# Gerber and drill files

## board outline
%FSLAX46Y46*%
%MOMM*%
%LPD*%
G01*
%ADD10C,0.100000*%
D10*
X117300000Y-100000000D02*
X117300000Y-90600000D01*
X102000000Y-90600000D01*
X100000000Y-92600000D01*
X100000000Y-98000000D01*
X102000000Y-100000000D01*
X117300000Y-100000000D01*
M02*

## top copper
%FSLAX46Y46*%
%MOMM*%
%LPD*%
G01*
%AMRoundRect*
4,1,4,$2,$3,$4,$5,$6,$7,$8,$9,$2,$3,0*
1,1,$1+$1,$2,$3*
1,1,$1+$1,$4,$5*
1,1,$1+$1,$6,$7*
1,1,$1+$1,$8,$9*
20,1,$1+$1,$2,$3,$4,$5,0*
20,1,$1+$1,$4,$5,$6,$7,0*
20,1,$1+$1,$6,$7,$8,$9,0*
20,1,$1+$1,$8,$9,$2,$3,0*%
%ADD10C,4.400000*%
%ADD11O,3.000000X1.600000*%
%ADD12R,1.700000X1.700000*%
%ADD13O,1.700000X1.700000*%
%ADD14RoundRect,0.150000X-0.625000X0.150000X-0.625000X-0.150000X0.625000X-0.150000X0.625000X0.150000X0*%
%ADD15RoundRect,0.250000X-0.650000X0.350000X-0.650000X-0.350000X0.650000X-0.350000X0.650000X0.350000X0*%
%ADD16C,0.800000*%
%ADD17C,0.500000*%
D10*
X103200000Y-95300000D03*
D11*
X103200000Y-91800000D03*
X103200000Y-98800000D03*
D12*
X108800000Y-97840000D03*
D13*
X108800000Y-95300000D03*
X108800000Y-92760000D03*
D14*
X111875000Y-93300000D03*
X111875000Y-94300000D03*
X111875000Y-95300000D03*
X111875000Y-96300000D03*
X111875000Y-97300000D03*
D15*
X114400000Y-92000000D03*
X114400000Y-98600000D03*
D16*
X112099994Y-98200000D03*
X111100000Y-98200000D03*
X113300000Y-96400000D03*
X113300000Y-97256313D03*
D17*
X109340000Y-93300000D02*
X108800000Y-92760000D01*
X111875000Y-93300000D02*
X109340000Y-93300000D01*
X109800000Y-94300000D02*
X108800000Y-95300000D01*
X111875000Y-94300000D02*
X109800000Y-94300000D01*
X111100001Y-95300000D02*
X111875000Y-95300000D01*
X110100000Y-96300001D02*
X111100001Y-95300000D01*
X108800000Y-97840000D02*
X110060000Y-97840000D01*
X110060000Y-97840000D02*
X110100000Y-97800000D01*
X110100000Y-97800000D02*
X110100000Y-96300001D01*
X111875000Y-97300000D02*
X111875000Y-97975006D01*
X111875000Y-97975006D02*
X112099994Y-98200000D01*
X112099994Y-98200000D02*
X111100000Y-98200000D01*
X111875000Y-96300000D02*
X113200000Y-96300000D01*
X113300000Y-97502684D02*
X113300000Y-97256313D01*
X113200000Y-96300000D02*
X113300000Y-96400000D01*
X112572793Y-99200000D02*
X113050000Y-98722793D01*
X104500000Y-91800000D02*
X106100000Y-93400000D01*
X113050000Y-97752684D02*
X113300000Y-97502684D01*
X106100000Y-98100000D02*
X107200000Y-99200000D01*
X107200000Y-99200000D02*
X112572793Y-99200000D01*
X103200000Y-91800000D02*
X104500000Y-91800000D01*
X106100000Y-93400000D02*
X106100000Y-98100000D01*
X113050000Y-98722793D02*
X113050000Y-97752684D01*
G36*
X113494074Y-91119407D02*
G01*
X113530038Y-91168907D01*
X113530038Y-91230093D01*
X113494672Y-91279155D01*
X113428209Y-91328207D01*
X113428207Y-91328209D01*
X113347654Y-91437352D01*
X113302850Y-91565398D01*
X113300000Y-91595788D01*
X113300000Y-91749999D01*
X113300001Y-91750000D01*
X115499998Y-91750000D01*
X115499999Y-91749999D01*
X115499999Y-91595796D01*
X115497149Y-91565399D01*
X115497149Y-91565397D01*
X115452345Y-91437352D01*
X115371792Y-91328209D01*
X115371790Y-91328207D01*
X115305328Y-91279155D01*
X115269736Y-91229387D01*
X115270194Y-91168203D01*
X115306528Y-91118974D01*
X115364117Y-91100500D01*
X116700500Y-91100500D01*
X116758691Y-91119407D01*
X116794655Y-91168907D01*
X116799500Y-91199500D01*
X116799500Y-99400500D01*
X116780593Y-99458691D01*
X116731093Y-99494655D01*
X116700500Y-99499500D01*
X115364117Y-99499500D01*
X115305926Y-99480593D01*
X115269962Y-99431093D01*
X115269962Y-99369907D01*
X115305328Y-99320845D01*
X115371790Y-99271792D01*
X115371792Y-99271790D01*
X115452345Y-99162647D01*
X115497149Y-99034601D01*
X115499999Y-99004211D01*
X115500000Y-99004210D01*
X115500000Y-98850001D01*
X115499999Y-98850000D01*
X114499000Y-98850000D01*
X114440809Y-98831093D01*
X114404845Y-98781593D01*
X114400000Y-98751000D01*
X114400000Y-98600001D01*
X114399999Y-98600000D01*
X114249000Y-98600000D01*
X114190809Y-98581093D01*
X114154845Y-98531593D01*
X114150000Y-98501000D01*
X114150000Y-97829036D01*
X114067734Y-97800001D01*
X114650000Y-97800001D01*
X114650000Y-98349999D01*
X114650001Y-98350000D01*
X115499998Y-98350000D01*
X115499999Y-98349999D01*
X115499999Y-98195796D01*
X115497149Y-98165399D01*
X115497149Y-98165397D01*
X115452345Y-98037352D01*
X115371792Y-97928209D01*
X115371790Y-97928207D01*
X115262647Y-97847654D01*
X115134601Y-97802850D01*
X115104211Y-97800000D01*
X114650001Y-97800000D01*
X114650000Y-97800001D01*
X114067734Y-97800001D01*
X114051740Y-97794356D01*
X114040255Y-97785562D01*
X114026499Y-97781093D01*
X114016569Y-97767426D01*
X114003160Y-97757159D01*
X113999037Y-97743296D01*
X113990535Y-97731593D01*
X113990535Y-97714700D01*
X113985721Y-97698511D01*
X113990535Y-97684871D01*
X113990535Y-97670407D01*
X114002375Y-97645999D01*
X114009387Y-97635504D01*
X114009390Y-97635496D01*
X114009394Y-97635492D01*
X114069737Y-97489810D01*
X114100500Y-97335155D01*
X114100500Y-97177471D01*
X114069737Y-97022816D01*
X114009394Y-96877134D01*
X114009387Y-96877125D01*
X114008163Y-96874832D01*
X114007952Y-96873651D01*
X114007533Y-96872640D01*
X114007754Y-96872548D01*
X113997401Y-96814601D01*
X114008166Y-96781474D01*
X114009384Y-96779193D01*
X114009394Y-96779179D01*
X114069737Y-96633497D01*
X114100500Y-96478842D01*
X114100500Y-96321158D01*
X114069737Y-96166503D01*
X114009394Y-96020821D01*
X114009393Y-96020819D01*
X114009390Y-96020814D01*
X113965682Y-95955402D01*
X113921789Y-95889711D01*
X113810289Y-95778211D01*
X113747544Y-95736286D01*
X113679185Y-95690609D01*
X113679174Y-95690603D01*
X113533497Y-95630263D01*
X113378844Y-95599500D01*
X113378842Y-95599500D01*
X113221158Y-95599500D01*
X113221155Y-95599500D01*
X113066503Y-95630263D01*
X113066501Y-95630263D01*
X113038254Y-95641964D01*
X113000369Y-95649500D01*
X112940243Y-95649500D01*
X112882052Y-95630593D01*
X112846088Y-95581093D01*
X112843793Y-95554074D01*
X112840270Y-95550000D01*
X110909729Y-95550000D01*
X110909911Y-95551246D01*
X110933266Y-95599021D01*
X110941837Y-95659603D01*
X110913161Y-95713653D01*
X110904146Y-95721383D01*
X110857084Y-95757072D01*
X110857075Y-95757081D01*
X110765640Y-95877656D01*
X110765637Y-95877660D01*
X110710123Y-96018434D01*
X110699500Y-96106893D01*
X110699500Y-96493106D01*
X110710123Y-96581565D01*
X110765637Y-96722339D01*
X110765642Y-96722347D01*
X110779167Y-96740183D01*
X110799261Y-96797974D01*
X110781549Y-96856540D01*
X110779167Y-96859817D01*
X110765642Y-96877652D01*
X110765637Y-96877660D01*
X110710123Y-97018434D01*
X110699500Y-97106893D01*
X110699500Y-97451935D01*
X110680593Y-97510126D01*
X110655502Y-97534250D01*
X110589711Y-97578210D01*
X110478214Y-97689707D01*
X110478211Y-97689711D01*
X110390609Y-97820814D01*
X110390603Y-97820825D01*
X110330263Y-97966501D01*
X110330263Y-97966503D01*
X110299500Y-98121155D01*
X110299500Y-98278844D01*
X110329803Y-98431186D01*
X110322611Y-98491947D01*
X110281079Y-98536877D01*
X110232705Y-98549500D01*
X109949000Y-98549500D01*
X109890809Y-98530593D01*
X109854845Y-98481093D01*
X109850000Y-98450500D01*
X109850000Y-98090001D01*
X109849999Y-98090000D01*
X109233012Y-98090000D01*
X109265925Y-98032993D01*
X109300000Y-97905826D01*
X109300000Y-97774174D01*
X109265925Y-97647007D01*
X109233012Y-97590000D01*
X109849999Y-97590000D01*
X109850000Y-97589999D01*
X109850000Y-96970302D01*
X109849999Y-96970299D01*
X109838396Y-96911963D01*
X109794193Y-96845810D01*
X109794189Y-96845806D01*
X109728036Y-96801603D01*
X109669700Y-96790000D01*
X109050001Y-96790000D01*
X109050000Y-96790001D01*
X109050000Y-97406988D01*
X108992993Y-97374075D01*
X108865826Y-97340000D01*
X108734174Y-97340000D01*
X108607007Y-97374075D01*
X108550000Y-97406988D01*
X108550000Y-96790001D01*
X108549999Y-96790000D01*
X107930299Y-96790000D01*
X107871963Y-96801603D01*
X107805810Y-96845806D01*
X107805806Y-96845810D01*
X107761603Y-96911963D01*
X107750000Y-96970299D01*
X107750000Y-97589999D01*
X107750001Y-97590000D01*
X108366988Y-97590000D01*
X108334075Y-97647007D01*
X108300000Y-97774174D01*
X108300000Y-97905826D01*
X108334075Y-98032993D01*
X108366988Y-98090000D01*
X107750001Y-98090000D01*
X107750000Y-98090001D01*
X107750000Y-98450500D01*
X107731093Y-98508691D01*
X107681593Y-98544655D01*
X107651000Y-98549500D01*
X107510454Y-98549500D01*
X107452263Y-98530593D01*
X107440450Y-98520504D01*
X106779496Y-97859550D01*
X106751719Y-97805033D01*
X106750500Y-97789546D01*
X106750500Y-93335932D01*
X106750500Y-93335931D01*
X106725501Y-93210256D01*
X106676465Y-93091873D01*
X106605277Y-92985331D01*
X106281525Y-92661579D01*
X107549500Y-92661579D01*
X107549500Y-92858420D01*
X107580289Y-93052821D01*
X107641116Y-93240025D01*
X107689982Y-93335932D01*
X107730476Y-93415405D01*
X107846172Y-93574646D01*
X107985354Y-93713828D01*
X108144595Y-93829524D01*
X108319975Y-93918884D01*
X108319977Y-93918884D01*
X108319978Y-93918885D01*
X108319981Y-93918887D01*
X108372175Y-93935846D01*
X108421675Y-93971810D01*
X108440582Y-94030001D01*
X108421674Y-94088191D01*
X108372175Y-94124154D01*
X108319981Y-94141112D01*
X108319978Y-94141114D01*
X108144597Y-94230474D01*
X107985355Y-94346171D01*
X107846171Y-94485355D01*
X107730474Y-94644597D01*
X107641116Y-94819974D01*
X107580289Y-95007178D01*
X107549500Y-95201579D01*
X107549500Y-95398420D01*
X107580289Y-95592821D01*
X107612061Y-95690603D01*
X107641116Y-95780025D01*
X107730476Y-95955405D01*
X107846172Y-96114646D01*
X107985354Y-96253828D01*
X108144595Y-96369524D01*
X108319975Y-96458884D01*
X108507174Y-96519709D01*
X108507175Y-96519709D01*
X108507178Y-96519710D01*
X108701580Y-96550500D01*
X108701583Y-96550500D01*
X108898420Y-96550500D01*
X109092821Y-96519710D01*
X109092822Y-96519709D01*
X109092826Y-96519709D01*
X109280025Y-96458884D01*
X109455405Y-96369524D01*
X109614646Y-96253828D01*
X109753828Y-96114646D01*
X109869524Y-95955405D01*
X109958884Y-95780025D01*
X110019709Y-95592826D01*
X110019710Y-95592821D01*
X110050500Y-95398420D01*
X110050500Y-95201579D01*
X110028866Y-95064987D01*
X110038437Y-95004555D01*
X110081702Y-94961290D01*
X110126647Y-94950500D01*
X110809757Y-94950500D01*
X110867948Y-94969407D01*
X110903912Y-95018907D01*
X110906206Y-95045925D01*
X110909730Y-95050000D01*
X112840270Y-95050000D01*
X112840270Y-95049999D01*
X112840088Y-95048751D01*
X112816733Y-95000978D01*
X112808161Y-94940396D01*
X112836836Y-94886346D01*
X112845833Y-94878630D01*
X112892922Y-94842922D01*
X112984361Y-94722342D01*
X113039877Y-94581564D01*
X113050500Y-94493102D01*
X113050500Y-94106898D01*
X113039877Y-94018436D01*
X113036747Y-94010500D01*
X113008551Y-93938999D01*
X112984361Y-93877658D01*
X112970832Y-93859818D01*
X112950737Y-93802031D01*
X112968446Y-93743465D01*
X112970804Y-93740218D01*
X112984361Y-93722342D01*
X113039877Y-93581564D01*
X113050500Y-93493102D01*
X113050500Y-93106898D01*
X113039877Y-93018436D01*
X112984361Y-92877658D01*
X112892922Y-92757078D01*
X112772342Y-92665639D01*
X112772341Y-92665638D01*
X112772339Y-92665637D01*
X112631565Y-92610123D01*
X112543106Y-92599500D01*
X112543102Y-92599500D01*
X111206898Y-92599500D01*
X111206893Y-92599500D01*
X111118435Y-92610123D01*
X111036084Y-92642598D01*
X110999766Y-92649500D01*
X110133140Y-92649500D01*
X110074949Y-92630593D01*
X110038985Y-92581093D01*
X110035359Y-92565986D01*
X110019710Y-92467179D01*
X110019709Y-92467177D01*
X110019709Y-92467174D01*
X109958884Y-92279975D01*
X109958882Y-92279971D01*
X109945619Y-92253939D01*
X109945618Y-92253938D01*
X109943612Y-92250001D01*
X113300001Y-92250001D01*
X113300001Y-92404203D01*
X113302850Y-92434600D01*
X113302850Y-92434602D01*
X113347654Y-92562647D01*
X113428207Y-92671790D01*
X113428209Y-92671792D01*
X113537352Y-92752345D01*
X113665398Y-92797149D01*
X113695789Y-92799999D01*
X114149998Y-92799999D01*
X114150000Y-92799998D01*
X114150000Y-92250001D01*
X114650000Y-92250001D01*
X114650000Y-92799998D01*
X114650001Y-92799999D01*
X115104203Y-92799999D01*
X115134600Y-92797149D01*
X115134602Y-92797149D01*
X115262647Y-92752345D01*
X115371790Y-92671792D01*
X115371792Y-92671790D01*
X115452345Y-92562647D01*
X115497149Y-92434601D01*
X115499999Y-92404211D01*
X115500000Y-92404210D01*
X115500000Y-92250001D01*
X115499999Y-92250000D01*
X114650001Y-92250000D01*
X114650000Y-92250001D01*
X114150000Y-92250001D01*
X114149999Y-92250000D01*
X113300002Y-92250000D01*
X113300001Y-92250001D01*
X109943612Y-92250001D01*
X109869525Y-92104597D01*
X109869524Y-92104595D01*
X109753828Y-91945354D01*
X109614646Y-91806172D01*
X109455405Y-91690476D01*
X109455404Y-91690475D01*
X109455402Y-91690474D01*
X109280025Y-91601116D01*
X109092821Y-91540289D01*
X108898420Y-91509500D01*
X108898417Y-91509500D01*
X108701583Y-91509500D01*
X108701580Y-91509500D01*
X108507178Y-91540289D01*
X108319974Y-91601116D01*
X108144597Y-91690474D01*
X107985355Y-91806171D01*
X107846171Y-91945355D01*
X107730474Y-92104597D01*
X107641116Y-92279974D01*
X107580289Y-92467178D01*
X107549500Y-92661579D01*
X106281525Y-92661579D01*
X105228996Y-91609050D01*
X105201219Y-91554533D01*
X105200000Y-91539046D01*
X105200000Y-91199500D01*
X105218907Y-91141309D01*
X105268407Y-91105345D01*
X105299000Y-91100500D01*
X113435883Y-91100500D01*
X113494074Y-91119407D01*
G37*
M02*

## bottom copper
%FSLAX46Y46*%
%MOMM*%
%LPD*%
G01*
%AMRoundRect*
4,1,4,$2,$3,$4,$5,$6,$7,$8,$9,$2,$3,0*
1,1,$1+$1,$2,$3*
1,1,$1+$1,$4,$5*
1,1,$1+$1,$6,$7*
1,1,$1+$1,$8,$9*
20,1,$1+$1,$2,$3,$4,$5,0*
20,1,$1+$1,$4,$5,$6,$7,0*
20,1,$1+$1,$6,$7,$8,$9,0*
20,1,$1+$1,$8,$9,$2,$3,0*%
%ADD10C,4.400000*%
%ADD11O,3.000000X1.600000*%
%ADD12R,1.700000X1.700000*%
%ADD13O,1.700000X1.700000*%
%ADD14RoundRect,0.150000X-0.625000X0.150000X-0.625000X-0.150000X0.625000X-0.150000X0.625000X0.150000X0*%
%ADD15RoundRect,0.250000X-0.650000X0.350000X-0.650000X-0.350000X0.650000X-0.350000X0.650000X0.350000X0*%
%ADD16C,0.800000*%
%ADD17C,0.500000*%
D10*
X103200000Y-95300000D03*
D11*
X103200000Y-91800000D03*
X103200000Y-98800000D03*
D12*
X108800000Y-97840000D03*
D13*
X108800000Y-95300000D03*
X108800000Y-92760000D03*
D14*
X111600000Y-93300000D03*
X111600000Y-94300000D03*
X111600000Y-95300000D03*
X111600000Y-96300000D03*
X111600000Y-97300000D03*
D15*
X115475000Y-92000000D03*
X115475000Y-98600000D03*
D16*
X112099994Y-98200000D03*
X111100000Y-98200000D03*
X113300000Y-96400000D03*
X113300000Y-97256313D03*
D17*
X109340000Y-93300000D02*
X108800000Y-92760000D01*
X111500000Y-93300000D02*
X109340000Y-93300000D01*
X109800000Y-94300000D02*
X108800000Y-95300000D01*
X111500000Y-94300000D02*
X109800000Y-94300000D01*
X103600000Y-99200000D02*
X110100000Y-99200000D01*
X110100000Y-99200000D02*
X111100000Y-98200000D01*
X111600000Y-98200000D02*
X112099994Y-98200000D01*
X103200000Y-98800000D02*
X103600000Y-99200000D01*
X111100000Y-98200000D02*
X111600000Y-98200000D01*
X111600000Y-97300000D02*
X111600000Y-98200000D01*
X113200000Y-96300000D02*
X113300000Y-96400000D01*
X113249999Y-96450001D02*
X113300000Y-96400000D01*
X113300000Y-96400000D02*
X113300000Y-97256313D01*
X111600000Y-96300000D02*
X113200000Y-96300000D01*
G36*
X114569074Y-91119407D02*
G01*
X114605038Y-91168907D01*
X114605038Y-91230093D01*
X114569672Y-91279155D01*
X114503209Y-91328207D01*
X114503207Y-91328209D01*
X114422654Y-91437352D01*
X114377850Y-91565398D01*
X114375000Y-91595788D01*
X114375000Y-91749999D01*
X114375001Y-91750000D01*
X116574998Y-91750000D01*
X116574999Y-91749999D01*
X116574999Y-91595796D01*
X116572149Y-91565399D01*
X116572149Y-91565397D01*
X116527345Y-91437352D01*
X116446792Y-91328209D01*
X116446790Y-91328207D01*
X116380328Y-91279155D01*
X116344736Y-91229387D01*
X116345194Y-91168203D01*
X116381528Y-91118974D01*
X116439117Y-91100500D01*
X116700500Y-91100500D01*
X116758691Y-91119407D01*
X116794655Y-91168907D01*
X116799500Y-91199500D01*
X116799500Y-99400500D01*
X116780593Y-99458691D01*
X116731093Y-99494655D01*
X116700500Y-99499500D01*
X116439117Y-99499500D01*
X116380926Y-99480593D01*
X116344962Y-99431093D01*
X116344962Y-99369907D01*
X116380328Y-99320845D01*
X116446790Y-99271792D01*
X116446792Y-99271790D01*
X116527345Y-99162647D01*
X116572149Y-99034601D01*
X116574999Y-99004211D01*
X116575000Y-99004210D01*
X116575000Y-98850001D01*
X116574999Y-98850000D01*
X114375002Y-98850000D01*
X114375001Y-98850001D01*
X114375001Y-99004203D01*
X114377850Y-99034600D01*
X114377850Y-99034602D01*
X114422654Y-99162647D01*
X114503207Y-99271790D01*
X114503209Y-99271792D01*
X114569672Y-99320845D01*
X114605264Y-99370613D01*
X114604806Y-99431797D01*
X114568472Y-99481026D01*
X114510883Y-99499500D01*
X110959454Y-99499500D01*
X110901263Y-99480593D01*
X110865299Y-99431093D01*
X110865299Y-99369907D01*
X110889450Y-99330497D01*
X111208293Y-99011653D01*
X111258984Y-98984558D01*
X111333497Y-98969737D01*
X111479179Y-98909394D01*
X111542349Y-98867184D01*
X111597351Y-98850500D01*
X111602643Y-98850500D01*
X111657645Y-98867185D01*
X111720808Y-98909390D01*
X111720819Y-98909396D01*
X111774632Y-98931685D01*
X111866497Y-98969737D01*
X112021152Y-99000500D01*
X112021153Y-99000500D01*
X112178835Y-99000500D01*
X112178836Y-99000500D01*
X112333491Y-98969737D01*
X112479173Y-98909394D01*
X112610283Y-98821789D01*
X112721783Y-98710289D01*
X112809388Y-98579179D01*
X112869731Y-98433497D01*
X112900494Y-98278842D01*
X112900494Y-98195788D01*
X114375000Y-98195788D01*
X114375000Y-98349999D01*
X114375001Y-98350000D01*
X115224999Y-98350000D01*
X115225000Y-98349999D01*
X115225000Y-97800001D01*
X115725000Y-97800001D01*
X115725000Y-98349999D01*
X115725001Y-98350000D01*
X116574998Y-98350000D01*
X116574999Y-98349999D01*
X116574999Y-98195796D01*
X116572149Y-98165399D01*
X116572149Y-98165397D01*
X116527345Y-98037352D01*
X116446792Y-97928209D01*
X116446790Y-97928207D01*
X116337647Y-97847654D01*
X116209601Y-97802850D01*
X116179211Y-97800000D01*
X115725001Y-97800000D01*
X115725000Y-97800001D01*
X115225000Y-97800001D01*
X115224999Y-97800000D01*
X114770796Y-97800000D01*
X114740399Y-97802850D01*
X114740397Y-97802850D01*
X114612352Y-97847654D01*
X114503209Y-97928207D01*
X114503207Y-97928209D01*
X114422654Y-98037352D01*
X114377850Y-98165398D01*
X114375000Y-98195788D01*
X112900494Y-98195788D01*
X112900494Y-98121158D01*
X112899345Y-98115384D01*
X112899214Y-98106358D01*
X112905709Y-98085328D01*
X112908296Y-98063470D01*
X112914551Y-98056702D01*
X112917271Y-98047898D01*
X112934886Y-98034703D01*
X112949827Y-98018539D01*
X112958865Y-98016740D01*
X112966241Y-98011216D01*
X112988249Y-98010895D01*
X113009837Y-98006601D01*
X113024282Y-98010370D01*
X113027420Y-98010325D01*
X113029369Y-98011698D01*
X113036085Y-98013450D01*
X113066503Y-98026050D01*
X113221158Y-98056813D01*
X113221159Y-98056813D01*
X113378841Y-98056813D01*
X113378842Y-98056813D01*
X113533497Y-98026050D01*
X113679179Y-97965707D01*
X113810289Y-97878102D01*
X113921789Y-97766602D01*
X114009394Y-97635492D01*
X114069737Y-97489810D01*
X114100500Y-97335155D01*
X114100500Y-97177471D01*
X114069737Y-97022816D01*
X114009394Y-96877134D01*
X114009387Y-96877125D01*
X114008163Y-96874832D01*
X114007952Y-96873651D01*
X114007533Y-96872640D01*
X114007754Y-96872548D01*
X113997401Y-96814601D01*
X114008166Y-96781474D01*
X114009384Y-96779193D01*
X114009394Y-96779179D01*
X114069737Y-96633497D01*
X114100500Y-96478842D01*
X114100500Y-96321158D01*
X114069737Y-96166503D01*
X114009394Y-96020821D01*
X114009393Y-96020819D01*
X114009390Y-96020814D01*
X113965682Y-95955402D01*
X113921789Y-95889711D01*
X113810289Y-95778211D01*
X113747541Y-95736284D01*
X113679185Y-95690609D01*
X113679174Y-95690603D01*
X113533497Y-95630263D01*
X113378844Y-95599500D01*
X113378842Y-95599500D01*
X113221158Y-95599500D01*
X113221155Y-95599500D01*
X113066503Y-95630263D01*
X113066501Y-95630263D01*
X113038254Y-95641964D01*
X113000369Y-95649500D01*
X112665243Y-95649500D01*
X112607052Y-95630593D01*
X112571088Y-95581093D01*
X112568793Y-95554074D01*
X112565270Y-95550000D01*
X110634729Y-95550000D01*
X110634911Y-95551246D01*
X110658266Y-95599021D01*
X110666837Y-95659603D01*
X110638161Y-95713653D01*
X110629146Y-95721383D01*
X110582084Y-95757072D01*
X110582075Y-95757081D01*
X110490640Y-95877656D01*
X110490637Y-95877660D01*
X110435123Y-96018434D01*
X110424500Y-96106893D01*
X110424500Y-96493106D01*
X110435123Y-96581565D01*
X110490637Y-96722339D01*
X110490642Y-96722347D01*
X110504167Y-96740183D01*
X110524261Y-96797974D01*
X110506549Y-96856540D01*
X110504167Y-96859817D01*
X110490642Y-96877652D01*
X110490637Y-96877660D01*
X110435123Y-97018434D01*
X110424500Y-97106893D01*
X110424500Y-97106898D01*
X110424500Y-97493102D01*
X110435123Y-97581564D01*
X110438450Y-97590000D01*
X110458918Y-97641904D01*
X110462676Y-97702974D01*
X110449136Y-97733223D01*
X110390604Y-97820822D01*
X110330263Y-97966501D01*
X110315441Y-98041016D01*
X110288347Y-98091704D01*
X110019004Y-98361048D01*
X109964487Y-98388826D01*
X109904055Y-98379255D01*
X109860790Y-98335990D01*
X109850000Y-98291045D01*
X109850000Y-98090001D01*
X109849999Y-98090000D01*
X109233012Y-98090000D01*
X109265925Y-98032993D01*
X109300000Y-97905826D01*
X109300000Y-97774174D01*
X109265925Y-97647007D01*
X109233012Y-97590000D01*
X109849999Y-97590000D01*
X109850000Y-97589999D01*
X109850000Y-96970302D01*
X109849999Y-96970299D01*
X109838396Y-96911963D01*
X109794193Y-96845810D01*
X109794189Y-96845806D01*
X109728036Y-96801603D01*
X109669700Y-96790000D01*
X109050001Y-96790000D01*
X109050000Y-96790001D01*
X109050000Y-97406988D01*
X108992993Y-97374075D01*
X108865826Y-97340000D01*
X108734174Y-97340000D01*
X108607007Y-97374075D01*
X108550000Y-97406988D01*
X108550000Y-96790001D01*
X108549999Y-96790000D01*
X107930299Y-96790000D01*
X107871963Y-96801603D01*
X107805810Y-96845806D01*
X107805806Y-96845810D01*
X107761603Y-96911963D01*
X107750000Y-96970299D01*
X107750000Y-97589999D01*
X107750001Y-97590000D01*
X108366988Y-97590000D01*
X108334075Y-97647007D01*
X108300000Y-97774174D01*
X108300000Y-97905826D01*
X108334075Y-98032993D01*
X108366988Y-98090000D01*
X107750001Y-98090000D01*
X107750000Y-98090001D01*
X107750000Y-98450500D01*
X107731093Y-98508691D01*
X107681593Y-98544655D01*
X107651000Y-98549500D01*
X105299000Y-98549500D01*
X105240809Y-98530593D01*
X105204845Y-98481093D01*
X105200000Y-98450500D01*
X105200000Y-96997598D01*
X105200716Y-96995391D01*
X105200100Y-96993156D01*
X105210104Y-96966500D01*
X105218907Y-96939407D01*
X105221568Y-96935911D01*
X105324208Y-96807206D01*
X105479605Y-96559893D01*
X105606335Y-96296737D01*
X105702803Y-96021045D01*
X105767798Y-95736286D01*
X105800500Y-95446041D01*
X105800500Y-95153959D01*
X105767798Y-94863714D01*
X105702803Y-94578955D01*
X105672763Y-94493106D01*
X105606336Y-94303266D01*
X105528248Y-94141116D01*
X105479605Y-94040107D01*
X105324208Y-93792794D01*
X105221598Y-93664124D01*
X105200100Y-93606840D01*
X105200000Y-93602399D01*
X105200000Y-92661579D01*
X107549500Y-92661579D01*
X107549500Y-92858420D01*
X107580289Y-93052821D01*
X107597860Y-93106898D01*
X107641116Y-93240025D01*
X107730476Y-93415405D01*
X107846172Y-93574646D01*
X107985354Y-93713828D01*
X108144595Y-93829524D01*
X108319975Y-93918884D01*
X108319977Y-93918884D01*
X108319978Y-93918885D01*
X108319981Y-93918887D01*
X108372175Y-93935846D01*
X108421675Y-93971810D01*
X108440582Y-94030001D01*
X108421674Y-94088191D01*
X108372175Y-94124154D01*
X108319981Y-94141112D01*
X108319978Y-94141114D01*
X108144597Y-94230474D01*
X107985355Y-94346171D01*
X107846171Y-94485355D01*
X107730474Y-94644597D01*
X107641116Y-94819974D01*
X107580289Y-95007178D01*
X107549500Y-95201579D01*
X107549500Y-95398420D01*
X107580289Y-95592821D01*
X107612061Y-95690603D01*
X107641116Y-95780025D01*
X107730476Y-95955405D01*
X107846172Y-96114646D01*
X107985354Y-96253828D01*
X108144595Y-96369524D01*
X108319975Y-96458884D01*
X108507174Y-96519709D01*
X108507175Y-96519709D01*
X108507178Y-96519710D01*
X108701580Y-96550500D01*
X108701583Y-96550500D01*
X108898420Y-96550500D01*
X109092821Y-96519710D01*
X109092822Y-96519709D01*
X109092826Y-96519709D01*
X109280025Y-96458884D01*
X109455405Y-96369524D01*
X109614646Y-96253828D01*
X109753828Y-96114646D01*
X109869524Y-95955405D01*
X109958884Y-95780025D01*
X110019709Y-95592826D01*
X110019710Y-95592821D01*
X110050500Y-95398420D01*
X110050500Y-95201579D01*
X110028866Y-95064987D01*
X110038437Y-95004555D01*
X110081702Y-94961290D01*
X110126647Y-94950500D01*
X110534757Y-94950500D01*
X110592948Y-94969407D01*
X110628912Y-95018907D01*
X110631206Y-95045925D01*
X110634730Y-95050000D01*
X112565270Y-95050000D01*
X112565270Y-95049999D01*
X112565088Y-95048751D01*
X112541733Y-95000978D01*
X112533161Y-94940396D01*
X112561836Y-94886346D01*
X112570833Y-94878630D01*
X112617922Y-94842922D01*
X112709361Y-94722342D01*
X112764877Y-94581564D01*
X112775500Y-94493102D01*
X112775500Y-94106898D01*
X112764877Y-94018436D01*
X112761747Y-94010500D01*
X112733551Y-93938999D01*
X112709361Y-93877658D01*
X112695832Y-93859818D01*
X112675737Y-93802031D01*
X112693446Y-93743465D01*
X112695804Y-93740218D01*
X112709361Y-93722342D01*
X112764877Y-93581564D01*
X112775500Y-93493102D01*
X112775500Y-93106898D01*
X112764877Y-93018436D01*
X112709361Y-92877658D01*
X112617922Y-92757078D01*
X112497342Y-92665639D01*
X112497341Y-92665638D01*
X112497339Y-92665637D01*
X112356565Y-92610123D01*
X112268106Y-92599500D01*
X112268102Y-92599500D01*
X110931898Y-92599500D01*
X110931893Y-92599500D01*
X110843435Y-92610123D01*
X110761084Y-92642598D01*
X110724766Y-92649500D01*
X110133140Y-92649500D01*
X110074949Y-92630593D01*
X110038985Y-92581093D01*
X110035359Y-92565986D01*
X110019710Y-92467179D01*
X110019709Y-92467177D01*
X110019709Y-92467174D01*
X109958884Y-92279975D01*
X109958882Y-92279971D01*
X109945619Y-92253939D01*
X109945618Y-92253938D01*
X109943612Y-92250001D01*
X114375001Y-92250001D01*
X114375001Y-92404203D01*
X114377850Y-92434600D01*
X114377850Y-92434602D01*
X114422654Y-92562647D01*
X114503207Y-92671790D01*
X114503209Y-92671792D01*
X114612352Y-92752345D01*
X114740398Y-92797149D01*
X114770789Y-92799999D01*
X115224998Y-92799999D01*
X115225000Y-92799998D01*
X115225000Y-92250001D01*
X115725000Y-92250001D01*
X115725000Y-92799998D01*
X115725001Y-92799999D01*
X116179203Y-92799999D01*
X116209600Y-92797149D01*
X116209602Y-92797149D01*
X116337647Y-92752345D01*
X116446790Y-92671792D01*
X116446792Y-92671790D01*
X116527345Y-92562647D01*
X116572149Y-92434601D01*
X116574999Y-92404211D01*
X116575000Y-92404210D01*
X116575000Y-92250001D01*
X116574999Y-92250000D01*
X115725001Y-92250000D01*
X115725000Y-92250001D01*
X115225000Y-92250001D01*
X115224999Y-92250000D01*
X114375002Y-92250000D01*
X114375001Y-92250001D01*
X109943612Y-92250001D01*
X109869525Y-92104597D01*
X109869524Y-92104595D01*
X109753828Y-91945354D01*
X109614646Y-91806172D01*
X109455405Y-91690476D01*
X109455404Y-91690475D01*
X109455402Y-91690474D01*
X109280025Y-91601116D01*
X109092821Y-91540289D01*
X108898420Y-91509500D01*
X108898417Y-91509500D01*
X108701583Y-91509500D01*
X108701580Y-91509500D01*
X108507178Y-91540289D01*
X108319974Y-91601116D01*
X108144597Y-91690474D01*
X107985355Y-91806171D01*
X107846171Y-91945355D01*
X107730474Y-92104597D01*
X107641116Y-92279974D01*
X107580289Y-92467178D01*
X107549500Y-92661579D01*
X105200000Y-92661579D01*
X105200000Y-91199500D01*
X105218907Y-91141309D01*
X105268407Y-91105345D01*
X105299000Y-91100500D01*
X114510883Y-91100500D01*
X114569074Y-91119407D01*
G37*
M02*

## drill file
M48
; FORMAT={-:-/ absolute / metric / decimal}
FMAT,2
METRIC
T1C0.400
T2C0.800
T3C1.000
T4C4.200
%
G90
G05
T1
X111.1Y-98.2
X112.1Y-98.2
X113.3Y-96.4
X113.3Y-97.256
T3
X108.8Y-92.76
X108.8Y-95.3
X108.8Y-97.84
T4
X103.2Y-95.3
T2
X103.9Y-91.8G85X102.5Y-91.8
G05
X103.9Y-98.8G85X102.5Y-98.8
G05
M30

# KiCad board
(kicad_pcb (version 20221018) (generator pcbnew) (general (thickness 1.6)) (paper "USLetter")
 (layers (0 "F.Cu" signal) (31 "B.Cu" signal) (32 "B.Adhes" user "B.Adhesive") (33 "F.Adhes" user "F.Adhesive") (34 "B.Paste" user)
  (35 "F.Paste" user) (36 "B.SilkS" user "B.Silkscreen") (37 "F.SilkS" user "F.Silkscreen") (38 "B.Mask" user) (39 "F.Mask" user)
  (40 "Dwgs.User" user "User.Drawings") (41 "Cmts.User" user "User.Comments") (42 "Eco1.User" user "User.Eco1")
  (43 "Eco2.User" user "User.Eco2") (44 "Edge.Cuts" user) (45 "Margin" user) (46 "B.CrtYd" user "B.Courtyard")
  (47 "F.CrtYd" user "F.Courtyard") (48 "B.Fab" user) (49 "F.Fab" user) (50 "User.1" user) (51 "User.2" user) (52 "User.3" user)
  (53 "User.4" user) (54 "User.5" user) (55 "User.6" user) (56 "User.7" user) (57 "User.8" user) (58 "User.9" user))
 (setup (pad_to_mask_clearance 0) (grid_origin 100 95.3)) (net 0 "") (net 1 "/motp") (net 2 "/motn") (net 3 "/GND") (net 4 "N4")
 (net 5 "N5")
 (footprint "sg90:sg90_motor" (layer "F.Cu") (at 103.2 95.3 180)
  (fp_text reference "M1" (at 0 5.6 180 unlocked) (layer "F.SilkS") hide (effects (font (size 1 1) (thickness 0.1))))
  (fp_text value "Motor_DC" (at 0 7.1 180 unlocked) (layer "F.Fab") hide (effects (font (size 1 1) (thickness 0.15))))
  (pad "" thru_hole circle (at 0 0 180) (size 4.4 4.4) (drill 4.2) (layers "*.Cu" "*.Mask"))
  (pad "1" thru_hole oval (at 0 3.5 180) (size 3 1.6) (drill oval 2.2 0.8) (layers "*.Cu" "*.Mask") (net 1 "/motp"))
  (pad "2" thru_hole oval (at 0 -3.5 180) (size 3 1.6) (drill oval 2.2 0.8) (layers "*.Cu" "*.Mask") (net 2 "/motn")))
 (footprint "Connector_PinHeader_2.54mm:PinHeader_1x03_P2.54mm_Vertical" (layer "F.Cu") (at 108.8 97.84 180)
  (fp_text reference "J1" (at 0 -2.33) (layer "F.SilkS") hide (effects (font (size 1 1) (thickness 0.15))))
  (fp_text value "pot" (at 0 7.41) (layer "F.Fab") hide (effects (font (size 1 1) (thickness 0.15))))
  (pad "1" thru_hole rect (at 0 0 180) (size 1.7 1.7) (drill 1) (layers "*.Cu" "*.Mask") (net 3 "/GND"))
  (pad "2" thru_hole oval (at 0 2.54 180) (size 1.7 1.7) (drill 1) (layers "*.Cu" "*.Mask") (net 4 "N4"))
  (pad "3" thru_hole oval (at 0 5.08 180) (size 1.7 1.7) (drill 1) (layers "*.Cu" "*.Mask") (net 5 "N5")))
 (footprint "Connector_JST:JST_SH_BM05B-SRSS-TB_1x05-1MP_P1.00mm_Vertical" (layer "F.Cu") (at 113.2 95.3 -90)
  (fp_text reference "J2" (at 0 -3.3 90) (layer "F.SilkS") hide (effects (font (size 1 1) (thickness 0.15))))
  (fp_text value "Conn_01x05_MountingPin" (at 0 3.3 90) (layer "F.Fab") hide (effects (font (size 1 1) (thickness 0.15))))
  (pad "1" smd roundrect (at -2 1.325 270) (size 0.6 1.55) (layers "F.Cu" "F.Paste" "F.Mask") (roundrect_rratio 0.25) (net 5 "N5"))
  (pad "2" smd roundrect (at -1 1.325 270) (size 0.6 1.55) (layers "F.Cu" "F.Paste" "F.Mask") (roundrect_rratio 0.25) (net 4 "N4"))
  (pad "3" smd roundrect (at 0 1.325 270) (size 0.6 1.55) (layers "F.Cu" "F.Paste" "F.Mask") (roundrect_rratio 0.25) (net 3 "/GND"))
  (pad "4" smd roundrect (at 1 1.325 270) (size 0.6 1.55) (layers "F.Cu" "F.Paste" "F.Mask") (roundrect_rratio 0.25) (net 1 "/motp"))
  (pad "5" smd roundrect (at 2 1.325 270) (size 0.6 1.55) (layers "F.Cu" "F.Paste" "F.Mask") (roundrect_rratio 0.25) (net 2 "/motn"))
  (pad "MP" smd roundrect (at -3.3 -1.2 270) (size 1.2 1.8) (layers "F.Cu" "F.Paste" "F.Mask") (roundrect_rratio 0.2083333333)
   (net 3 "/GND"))
  (pad "MP" smd roundrect (at 3.3 -1.2 270) (size 1.2 1.8) (layers "F.Cu" "F.Paste" "F.Mask") (roundrect_rratio 0.2083333333) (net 3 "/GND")))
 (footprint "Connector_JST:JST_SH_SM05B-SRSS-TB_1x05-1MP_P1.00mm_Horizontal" (layer "B.Cu") (at 113.6 95.3 -90)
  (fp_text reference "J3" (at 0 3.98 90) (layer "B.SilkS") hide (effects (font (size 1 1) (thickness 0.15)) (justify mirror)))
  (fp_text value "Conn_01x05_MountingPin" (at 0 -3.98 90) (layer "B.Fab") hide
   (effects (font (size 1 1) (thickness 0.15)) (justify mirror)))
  (pad "1" smd roundrect (at -2 2 270) (size 0.6 1.55) (layers "B.Cu" "B.Paste" "B.Mask") (roundrect_rratio 0.25) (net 5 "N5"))
  (pad "2" smd roundrect (at -1 2 270) (size 0.6 1.55) (layers "B.Cu" "B.Paste" "B.Mask") (roundrect_rratio 0.25) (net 4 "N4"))
  (pad "3" smd roundrect (at 0 2 270) (size 0.6 1.55) (layers "B.Cu" "B.Paste" "B.Mask") (roundrect_rratio 0.25) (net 3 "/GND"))
  (pad "4" smd roundrect (at 1 2 270) (size 0.6 1.55) (layers "B.Cu" "B.Paste" "B.Mask") (roundrect_rratio 0.25) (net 1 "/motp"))
  (pad "5" smd roundrect (at 2 2 270) (size 0.6 1.55) (layers "B.Cu" "B.Paste" "B.Mask") (roundrect_rratio 0.25) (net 2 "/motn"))
  (pad "MP" smd roundrect (at -3.3 -1.875 270) (size 1.2 1.8) (layers "B.Cu" "B.Paste" "B.Mask") (roundrect_rratio 0.2083333333)
   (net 3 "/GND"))
  (pad "MP" smd roundrect (at 3.3 -1.875 270) (size 1.2 1.8) (layers "B.Cu" "B.Paste" "B.Mask") (roundrect_rratio 0.2083333333)
   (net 3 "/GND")))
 (gr_poly
  (pts (xy 117.3 100) (xy 117.3 90.6) (xy 102 90.6) (xy 100 92.6) (xy 100 98) (xy 102 100)) (stroke (width 0.1) (type solid)) (fill none)
  (layer "Edge.Cuts"))
 (segment (start 109.34 93.3) (end 108.8 92.76) (width 0.5) (layer "F.Cu") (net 5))
 (segment (start 111.875 93.3) (end 109.34 93.3) (width 0.5) (layer "F.Cu") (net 5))
 (segment (start 109.34 93.3) (end 108.8 92.76) (width 0.5) (layer "B.Cu") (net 5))
 (segment (start 111.5 93.3) (end 109.34 93.3) (width 0.5) (layer "B.Cu") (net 5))
 (segment (start 109.8 94.3) (end 108.8 95.3) (width 0.5) (layer "F.Cu") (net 4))
 (segment (start 111.875 94.3) (end 109.8 94.3) (width 0.5) (layer "F.Cu") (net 4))
 (segment (start 109.8 94.3) (end 108.8 95.3) (width 0.5) (layer "B.Cu") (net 4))
 (segment (start 111.5 94.3) (end 109.8 94.3) (width 0.5) (layer "B.Cu") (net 4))
 (segment (start 111.100001 95.3) (end 111.875 95.3) (width 0.5) (layer "F.Cu") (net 3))
 (segment (start 110.1 96.300001) (end 111.100001 95.3) (width 0.5) (layer "F.Cu") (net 3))
 (segment (start 108.8 97.84) (end 110.06 97.84) (width 0.5) (layer "F.Cu") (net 3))
 (segment (start 110.06 97.84) (end 110.1 97.8) (width 0.5) (layer "F.Cu") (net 3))
 (segment (start 110.1 97.8) (end 110.1 96.300001) (width 0.5) (layer "F.Cu") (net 3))
 (segment (start 111.875 97.3) (end 111.875 97.975006) (width 0.5) (layer "F.Cu") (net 2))
 (segment (start 111.875 97.975006) (end 112.099994 98.2) (width 0.5) (layer "F.Cu") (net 2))
 (segment (start 112.099994 98.2) (end 111.1 98.2) (width 0.5) (layer "F.Cu") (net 2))
 (via (at 112.099994 98.2) (size 0.8) (drill 0.4) (layers "F.Cu" "B.Cu") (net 2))
 (via (at 111.1 98.2) (size 0.8) (drill 0.4) (layers "F.Cu" "B.Cu") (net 2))
 (segment (start 103.6 99.2) (end 110.1 99.2) (width 0.5) (layer "B.Cu") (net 2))
 (segment (start 110.1 99.2) (end 111.1 98.2) (width 0.5) (layer "B.Cu") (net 2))
 (segment (start 111.6 98.2) (end 112.099994 98.2) (width 0.5) (layer "B.Cu") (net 2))
 (segment (start 103.2 98.8) (end 103.6 99.2) (width 0.5) (layer "B.Cu") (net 2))
 (segment (start 111.1 98.2) (end 111.6 98.2) (width 0.5) (layer "B.Cu") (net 2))
 (segment (start 111.6 97.3) (end 111.6 98.2) (width 0.5) (layer "B.Cu") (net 2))
 (segment (start 111.875 96.3) (end 113.2 96.3) (width 0.5) (layer "F.Cu") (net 1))
 (segment (start 113.3 97.502684) (end 113.3 97.256313) (width 0.5) (layer "F.Cu") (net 1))
 (segment (start 113.2 96.3) (end 113.3 96.4) (width 0.5) (layer "F.Cu") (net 1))
 (segment (start 112.572793 99.2) (end 113.05 98.722793) (width 0.5) (layer "F.Cu") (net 1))
 (segment (start 104.5 91.8) (end 106.1 93.4) (width 0.5) (layer "F.Cu") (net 1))
 (segment (start 113.05 97.752684) (end 113.3 97.502684) (width 0.5) (layer "F.Cu") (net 1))
 (segment (start 106.1 98.1) (end 107.2 99.2) (width 0.5) (layer "F.Cu") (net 1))
 (segment (start 107.2 99.2) (end 112.572793 99.2) (width 0.5) (layer "F.Cu") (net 1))
 (segment (start 103.2 91.8) (end 104.5 91.8) (width 0.5) (layer "F.Cu") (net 1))
 (segment (start 106.1 93.4) (end 106.1 98.1) (width 0.5) (layer "F.Cu") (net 1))
 (segment (start 113.05 98.722793) (end 113.05 97.752684) (width 0.5) (layer "F.Cu") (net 1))
 (via (at 113.3 96.4) (size 0.8) (drill 0.4) (layers "F.Cu" "B.Cu") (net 1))
 (via (at 113.3 97.256313) (size 0.8) (drill 0.4) (layers "F.Cu" "B.Cu") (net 1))
 (segment (start 113.2 96.3) (end 113.3 96.4) (width 0.5) (layer "B.Cu") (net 1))
 (segment (start 113.249999 96.450001) (end 113.3 96.4) (width 0.5) (layer "B.Cu") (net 1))
 (segment (start 113.3 96.4) (end 113.3 97.256313) (width 0.5) (layer "B.Cu") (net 1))
 (segment (start 111.6 96.3) (end 113.2 96.3) (width 0.5) (layer "B.Cu") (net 1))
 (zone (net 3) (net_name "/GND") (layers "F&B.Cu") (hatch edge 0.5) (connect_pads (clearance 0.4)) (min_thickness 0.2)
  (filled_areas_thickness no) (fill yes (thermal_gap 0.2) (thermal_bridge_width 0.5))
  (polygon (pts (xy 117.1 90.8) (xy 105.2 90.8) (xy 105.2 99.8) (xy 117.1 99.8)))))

